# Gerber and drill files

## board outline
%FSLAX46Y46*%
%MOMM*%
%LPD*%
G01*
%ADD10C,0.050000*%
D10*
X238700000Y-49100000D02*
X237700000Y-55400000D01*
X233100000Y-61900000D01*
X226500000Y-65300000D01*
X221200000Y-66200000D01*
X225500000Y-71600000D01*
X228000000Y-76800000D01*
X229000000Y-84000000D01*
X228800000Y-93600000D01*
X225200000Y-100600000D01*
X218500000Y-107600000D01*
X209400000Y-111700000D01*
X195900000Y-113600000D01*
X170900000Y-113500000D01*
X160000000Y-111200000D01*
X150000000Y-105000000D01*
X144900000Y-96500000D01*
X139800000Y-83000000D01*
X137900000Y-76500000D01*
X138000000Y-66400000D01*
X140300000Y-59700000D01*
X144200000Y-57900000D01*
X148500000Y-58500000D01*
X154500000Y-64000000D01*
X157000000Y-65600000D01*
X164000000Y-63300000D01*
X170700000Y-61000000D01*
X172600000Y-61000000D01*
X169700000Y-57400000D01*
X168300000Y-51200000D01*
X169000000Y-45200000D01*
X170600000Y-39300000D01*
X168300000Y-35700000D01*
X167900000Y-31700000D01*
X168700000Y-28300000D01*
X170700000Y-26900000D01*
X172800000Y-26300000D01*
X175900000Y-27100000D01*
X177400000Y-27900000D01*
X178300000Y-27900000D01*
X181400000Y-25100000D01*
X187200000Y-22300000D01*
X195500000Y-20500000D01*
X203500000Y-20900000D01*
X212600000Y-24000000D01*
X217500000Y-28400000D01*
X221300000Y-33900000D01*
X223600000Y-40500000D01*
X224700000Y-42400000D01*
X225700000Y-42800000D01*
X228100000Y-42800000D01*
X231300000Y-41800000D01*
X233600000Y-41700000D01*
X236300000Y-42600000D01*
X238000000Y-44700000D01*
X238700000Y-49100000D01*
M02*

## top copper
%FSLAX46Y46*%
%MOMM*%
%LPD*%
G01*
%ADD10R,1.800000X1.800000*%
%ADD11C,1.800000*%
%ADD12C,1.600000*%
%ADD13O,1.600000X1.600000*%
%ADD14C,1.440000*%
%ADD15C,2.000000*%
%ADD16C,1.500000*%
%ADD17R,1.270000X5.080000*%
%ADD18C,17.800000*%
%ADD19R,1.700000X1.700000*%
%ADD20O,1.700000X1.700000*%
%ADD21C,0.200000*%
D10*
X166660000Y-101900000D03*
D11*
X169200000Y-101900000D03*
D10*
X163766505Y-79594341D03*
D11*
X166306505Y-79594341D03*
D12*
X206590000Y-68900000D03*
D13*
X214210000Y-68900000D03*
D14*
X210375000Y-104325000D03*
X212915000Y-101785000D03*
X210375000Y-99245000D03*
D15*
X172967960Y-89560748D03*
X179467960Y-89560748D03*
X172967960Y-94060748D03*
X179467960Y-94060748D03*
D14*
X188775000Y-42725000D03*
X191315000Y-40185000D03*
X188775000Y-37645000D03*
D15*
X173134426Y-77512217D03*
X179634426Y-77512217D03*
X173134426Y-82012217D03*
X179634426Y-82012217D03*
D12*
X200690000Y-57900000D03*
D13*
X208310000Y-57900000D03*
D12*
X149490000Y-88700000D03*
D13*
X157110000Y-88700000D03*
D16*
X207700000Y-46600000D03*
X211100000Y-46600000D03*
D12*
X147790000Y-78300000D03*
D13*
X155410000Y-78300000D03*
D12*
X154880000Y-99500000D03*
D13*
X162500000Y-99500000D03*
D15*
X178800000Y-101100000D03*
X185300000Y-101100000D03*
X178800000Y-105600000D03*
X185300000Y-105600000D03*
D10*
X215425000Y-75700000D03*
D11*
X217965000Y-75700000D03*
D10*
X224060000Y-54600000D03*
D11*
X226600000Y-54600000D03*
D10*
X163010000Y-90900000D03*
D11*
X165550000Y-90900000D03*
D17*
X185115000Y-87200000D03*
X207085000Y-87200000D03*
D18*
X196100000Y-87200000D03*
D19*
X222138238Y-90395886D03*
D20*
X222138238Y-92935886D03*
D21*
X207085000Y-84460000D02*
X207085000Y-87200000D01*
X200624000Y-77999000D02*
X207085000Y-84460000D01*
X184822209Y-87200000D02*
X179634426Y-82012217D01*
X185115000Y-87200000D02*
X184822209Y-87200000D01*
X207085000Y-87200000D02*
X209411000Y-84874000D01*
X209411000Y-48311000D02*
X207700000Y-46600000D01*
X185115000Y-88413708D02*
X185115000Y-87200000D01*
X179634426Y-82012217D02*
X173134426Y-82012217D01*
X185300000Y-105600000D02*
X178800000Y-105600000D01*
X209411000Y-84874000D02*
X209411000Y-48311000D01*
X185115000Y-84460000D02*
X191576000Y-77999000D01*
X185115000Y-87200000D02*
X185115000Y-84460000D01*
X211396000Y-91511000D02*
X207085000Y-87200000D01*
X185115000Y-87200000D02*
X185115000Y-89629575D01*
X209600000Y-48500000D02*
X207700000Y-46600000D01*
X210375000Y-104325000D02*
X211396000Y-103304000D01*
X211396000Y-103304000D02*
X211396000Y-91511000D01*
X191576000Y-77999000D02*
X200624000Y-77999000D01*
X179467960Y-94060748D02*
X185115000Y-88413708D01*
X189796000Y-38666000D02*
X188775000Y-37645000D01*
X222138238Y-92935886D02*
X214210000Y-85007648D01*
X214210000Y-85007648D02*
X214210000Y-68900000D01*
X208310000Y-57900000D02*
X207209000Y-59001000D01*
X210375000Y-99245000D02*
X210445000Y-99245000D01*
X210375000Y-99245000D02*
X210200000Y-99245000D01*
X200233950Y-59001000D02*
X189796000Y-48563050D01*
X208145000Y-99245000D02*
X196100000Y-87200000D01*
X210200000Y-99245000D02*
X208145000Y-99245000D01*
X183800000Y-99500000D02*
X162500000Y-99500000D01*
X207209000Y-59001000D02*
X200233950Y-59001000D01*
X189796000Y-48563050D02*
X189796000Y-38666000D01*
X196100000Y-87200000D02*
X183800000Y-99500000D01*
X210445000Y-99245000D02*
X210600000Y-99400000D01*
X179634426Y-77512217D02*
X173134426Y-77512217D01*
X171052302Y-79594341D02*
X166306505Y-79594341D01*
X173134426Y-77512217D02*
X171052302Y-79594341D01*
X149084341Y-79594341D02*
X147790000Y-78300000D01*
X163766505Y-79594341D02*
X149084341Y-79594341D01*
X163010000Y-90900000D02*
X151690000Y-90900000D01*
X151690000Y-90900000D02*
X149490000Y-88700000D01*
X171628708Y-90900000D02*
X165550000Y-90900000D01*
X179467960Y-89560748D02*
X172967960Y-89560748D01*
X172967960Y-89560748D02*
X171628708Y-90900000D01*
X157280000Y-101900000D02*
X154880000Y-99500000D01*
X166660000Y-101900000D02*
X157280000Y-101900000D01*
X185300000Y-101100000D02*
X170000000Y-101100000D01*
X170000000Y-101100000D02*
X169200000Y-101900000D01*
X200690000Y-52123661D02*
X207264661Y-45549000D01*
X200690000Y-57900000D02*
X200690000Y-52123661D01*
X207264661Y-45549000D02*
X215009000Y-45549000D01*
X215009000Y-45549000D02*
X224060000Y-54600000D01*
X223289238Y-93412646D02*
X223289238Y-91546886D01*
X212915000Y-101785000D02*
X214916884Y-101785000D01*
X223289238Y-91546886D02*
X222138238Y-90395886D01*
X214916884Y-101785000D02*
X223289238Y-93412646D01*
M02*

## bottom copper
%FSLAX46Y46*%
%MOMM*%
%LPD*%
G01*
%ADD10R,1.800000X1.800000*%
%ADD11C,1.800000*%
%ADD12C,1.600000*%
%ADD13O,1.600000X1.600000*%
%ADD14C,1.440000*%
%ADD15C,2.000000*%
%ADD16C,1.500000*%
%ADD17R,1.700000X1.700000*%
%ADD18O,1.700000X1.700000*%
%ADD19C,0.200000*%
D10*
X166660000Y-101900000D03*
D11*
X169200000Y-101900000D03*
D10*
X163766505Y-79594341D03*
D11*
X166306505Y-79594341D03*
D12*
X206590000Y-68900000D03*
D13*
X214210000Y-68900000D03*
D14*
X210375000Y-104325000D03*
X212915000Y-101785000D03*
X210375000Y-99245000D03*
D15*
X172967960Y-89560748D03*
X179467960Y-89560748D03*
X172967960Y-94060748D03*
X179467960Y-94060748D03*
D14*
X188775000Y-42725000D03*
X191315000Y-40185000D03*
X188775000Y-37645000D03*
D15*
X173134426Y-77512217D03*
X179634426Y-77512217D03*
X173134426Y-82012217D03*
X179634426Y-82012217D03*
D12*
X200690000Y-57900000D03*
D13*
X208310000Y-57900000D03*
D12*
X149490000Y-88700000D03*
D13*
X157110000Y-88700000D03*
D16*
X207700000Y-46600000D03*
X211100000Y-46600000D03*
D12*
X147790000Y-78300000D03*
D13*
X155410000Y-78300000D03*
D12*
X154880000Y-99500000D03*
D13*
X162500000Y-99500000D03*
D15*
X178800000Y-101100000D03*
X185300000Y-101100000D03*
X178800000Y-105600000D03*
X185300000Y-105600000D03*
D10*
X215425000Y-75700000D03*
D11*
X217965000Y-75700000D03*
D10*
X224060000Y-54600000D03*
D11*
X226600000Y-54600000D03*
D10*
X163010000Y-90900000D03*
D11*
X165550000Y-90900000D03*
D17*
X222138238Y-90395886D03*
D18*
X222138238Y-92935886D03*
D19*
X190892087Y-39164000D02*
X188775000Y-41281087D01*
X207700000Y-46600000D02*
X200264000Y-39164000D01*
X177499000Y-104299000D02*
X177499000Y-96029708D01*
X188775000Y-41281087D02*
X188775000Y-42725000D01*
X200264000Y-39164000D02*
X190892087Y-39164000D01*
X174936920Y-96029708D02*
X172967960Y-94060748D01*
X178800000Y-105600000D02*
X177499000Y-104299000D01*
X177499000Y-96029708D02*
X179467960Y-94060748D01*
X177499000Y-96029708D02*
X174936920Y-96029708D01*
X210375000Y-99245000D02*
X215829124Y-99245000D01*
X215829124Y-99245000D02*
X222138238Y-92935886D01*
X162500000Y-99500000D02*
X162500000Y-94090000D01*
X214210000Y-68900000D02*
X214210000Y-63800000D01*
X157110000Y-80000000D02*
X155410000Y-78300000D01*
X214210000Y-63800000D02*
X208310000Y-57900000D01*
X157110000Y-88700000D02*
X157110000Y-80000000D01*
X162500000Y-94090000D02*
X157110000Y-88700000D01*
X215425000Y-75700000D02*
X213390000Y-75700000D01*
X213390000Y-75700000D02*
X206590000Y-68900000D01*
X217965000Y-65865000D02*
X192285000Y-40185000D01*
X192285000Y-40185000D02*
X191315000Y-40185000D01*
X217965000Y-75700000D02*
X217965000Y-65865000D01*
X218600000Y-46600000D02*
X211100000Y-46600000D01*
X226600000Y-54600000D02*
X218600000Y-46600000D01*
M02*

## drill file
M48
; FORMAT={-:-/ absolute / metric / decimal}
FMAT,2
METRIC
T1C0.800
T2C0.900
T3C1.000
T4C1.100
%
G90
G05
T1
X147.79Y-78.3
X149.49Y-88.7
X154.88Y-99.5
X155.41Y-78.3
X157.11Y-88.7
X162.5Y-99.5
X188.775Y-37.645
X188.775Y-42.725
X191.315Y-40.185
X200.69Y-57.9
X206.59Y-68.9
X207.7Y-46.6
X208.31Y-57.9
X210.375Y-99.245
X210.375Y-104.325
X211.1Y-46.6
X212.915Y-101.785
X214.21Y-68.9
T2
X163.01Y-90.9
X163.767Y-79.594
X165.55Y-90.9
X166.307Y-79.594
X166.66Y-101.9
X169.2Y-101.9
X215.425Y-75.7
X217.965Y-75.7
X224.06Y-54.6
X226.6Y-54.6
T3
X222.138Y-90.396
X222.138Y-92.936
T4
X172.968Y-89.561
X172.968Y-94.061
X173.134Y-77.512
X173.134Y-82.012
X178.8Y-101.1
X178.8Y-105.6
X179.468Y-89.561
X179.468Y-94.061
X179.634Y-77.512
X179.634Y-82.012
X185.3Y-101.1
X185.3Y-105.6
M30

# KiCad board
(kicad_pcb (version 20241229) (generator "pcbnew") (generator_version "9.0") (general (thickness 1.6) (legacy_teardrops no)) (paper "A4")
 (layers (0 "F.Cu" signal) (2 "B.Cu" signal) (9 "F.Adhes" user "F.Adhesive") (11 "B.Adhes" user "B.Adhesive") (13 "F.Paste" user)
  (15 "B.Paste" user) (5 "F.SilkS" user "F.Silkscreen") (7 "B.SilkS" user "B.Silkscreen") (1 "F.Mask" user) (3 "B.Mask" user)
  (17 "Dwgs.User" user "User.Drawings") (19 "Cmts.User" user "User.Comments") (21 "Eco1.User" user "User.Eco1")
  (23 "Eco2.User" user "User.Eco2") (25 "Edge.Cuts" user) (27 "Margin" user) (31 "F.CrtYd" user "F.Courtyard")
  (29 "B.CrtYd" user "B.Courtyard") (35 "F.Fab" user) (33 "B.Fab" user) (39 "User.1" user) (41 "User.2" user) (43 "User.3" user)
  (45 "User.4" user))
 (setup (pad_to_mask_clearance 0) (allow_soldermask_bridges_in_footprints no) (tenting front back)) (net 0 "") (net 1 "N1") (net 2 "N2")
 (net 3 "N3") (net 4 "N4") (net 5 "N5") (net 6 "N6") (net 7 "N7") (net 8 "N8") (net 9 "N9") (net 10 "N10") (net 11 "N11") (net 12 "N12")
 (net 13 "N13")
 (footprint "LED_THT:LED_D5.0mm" (layer "F.Cu") (at 166.66 101.9)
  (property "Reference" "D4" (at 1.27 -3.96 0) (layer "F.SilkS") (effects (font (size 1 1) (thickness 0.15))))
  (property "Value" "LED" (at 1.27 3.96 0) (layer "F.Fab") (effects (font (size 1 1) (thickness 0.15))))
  (pad "1" thru_hole rect (at 0 0) (size 1.8 1.8) (drill 0.9) (layers "*.Cu" "*.Mask") (remove_unused_layers no) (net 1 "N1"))
  (pad "2" thru_hole circle (at 2.54 0) (size 1.8 1.8) (drill 0.9) (layers "*.Cu" "*.Mask") (remove_unused_layers no) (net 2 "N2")))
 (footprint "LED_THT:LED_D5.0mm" (layer "F.Cu") (at 163.766505 79.594341)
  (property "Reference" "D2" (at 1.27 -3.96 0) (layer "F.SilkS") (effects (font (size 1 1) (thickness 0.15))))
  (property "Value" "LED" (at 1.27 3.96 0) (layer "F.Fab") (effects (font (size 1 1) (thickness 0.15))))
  (pad "1" thru_hole rect (at 0 0) (size 1.8 1.8) (drill 0.9) (layers "*.Cu" "*.Mask") (remove_unused_layers no) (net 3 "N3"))
  (pad "2" thru_hole circle (at 2.54 0) (size 1.8 1.8) (drill 0.9) (layers "*.Cu" "*.Mask") (remove_unused_layers no) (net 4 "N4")))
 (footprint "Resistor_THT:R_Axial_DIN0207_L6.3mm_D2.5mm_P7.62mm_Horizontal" (layer "F.Cu") (at 206.59 68.9)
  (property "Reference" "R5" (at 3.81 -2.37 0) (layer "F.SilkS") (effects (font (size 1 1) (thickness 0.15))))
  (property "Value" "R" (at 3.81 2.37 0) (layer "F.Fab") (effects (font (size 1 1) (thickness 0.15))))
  (pad "1" thru_hole circle (at 0 0) (size 1.6 1.6) (drill 0.8) (layers "*.Cu" "*.Mask") (remove_unused_layers no) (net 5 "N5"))
  (pad "2" thru_hole oval (at 7.62 0) (size 1.6 1.6) (drill 0.8) (layers "*.Cu" "*.Mask") (remove_unused_layers no) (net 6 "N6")))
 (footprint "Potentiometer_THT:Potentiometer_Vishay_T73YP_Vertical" (layer "F.Cu") (at 210.375 104.325)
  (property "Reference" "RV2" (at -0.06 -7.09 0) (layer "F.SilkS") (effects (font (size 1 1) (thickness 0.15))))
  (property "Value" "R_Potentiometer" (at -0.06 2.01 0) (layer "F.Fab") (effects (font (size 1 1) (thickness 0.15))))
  (pad "1" thru_hole circle (at 0 0) (size 1.44 1.44) (drill 0.8) (layers "*.Cu" "*.Mask") (remove_unused_layers no) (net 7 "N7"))
  (pad "2" thru_hole circle (at 2.54 -2.54) (size 1.44 1.44) (drill 0.8) (layers "*.Cu" "*.Mask") (remove_unused_layers no) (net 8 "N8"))
  (pad "3" thru_hole circle (at 0 -5.08) (size 1.44 1.44) (drill 0.8) (layers "*.Cu" "*.Mask") (remove_unused_layers no) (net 6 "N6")))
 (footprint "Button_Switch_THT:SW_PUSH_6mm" (layer "F.Cu") (at 172.96796 89.560748)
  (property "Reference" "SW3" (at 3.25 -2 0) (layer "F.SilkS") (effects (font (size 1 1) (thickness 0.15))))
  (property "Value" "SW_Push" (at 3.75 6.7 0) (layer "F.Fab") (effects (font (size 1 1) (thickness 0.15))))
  (pad "1" thru_hole circle (at 0 0 90) (size 2 2) (drill 1.1) (layers "*.Cu" "*.Mask") (remove_unused_layers no) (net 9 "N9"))
  (pad "1" thru_hole circle (at 6.5 0 90) (size 2 2) (drill 1.1) (layers "*.Cu" "*.Mask") (remove_unused_layers no) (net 9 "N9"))
  (pad "2" thru_hole circle (at 0 4.5 90) (size 2 2) (drill 1.1) (layers "*.Cu" "*.Mask") (remove_unused_layers no) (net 7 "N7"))
  (pad "2" thru_hole circle (at 6.5 4.5 90) (size 2 2) (drill 1.1) (layers "*.Cu" "*.Mask") (remove_unused_layers no) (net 7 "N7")))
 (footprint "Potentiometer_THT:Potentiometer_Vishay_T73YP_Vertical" (layer "F.Cu") (at 188.775 42.725)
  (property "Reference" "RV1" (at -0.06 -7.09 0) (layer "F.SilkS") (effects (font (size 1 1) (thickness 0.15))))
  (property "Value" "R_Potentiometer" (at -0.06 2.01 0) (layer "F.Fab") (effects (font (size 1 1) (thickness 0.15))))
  (pad "1" thru_hole circle (at 0 0) (size 1.44 1.44) (drill 0.8) (layers "*.Cu" "*.Mask") (remove_unused_layers no) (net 7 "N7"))
  (pad "2" thru_hole circle (at 2.54 -2.54) (size 1.44 1.44) (drill 0.8) (layers "*.Cu" "*.Mask") (remove_unused_layers no) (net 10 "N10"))
  (pad "3" thru_hole circle (at 0 -5.08) (size 1.44 1.44) (drill 0.8) (layers "*.Cu" "*.Mask") (remove_unused_layers no) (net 6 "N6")))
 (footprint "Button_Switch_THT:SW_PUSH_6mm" (layer "F.Cu") (at 173.134426 77.512217)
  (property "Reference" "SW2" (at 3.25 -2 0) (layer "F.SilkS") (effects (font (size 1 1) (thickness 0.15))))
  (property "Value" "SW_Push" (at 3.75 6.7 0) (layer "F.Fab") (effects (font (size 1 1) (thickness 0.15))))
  (pad "1" thru_hole circle (at 0 0 90) (size 2 2) (drill 1.1) (layers "*.Cu" "*.Mask") (remove_unused_layers no) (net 4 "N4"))
  (pad "1" thru_hole circle (at 6.5 0 90) (size 2 2) (drill 1.1) (layers "*.Cu" "*.Mask") (remove_unused_layers no) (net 4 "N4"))
  (pad "2" thru_hole circle (at 0 4.5 90) (size 2 2) (drill 1.1) (layers "*.Cu" "*.Mask") (remove_unused_layers no) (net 7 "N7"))
  (pad "2" thru_hole circle (at 6.5 4.5 90) (size 2 2) (drill 1.1) (layers "*.Cu" "*.Mask") (remove_unused_layers no) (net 7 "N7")))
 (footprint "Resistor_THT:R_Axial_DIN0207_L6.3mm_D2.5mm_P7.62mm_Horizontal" (layer "F.Cu") (at 200.69 57.9)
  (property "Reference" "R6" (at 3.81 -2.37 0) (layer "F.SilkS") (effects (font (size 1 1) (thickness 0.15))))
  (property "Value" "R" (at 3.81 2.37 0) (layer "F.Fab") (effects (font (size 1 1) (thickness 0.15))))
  (pad "1" thru_hole circle (at 0 0) (size 1.6 1.6) (drill 0.8) (layers "*.Cu" "*.Mask") (remove_unused_layers no) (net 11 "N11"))
  (pad "2" thru_hole oval (at 7.62 0) (size 1.6 1.6) (drill 0.8) (layers "*.Cu" "*.Mask") (remove_unused_layers no) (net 6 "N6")))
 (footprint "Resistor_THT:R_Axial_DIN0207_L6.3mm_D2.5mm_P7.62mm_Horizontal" (layer "F.Cu") (at 149.49 88.7)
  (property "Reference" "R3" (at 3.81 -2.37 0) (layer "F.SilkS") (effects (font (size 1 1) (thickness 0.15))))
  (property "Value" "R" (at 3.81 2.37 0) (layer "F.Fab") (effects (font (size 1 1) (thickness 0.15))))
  (pad "1" thru_hole circle (at 0 0) (size 1.6 1.6) (drill 0.8) (layers "*.Cu" "*.Mask") (remove_unused_layers no) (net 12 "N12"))
  (pad "2" thru_hole oval (at 7.62 0) (size 1.6 1.6) (drill 0.8) (layers "*.Cu" "*.Mask") (remove_unused_layers no) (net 6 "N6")))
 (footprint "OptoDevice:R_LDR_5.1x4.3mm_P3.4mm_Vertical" (layer "F.Cu") (at 207.7 46.6)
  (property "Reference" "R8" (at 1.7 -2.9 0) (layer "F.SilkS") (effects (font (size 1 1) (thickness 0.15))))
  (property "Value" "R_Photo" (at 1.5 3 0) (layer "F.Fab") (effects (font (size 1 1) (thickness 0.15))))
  (pad "1" thru_hole circle (at 0 0) (size 1.5 1.5) (drill 0.8) (layers "*.Cu" "*.Mask") (remove_unused_layers no) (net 7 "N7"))
  (pad "2" thru_hole circle (at 3.4 0) (size 1.5 1.5) (drill 0.8) (layers "*.Cu" "*.Mask") (remove_unused_layers no) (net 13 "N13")))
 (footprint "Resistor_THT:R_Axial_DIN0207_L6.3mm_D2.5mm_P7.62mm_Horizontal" (layer "F.Cu") (at 147.79 78.3)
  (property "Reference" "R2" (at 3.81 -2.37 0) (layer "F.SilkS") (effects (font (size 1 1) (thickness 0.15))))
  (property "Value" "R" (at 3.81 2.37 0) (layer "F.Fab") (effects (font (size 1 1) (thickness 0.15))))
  (pad "1" thru_hole circle (at 0 0) (size 1.6 1.6) (drill 0.8) (layers "*.Cu" "*.Mask") (remove_unused_layers no) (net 3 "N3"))
  (pad "2" thru_hole oval (at 7.62 0) (size 1.6 1.6) (drill 0.8) (layers "*.Cu" "*.Mask") (remove_unused_layers no) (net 6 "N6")))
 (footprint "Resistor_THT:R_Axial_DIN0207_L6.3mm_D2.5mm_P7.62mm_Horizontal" (layer "F.Cu") (at 154.88 99.5)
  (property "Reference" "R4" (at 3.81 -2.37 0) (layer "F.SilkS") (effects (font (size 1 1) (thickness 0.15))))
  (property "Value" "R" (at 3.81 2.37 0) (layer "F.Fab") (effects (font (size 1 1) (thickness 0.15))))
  (pad "1" thru_hole circle (at 0 0) (size 1.6 1.6) (drill 0.8) (layers "*.Cu" "*.Mask") (remove_unused_layers no) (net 1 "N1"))
  (pad "2" thru_hole oval (at 7.62 0) (size 1.6 1.6) (drill 0.8) (layers "*.Cu" "*.Mask") (remove_unused_layers no) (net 6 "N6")))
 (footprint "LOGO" (layer "F.Cu") (at 189.1 67.6)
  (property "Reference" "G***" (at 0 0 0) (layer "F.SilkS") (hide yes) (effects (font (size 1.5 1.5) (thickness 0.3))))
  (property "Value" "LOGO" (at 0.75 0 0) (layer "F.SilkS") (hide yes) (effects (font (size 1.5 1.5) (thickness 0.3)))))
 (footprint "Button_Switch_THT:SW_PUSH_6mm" (layer "F.Cu") (at 178.8 101.1)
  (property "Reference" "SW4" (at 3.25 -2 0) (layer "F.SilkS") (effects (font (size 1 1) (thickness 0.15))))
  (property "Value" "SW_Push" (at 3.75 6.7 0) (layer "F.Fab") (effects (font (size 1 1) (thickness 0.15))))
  (pad "1" thru_hole circle (at 0 0 90) (size 2 2) (drill 1.1) (layers "*.Cu" "*.Mask") (remove_unused_layers no) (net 2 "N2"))
  (pad "1" thru_hole circle (at 6.5 0 90) (size 2 2) (drill 1.1) (layers "*.Cu" "*.Mask") (remove_unused_layers no) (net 2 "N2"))
  (pad "2" thru_hole circle (at 0 4.5 90) (size 2 2) (drill 1.1) (layers "*.Cu" "*.Mask") (remove_unused_layers no) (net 7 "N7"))
  (pad "2" thru_hole circle (at 6.5 4.5 90) (size 2 2) (drill 1.1) (layers "*.Cu" "*.Mask") (remove_unused_layers no) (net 7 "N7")))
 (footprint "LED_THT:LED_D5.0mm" (layer "F.Cu") (at 215.425 75.7)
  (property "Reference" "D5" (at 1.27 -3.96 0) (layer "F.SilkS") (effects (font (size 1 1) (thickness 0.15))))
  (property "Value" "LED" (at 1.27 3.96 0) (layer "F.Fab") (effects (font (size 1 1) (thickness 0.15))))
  (pad "1" thru_hole rect (at 0 0) (size 1.8 1.8) (drill 0.9) (layers "*.Cu" "*.Mask") (remove_unused_layers no) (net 5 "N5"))
  (pad "2" thru_hole circle (at 2.54 0) (size 1.8 1.8) (drill 0.9) (layers "*.Cu" "*.Mask") (remove_unused_layers no) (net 10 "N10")))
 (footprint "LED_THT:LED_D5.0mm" (layer "F.Cu") (at 224.06 54.6)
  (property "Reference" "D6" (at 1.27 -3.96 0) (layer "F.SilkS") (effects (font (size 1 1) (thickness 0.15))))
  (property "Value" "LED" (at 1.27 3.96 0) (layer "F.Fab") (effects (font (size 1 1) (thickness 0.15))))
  (pad "1" thru_hole rect (at 0 0) (size 1.8 1.8) (drill 0.9) (layers "*.Cu" "*.Mask") (remove_unused_layers no) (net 11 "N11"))
  (pad "2" thru_hole circle (at 2.54 0) (size 1.8 1.8) (drill 0.9) (layers "*.Cu" "*.Mask") (remove_unused_layers no) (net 13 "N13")))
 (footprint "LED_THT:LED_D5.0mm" (layer "F.Cu") (at 163.01 90.9)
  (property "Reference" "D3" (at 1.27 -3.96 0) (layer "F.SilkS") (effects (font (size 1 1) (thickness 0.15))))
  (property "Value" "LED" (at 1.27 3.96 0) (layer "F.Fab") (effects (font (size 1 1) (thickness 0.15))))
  (pad "1" thru_hole rect (at 0 0) (size 1.8 1.8) (drill 0.9) (layers "*.Cu" "*.Mask") (remove_unused_layers no) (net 12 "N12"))
  (pad "2" thru_hole circle (at 2.54 0) (size 1.8 1.8) (drill 0.9) (layers "*.Cu" "*.Mask") (remove_unused_layers no) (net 9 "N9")))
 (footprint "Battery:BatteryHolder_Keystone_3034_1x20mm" (layer "F.Cu") (at 196.1 87.2)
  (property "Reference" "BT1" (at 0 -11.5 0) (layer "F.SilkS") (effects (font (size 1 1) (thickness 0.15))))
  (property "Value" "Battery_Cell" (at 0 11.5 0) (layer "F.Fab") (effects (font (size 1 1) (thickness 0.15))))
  (pad "1" smd rect (at -10.985 0) (size 1.27 5.08) (layers "F.Cu" "F.Mask" "F.Paste") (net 7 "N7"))
  (pad "1" smd rect (at 10.985 0) (size 1.27 5.08) (layers "F.Cu" "F.Mask" "F.Paste") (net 7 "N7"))
  (pad "2" smd circle (at 0 0) (size 17.8 17.8) (layers "F.Cu" "F.Mask") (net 6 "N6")))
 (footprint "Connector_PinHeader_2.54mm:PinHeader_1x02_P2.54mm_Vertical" (layer "F.Cu") (at 222.138238 90.395886)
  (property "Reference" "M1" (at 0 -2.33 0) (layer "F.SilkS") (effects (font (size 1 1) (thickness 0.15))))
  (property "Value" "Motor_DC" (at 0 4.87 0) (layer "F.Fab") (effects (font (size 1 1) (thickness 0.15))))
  (pad "1" thru_hole rect (at 0 0) (size 1.7 1.7) (drill 1) (layers "*.Cu" "*.Mask") (remove_unused_layers no) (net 8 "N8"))
  (pad "2" thru_hole oval (at 0 2.54) (size 1.7 1.7) (drill 1) (layers "*.Cu" "*.Mask") (remove_unused_layers no) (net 6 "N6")))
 (gr_poly
  (pts (xy 238.7 49.1) (xy 237.7 55.4) (xy 233.1 61.9) (xy 226.5 65.3) (xy 221.2 66.2) (xy 225.5 71.6) (xy 228 76.8) (xy 229 84)
   (xy 228.8 93.6) (xy 225.2 100.6) (xy 218.5 107.6) (xy 209.4 111.7) (xy 195.9 113.6) (xy 170.9 113.5) (xy 160 111.2) (xy 150 105)
   (xy 144.9 96.5) (xy 139.8 83) (xy 137.9 76.5) (xy 138 66.4) (xy 140.3 59.7) (xy 144.2 57.9) (xy 148.5 58.5) (xy 154.5 64) (xy 157 65.6)
   (xy 164 63.3) (xy 170.7 61) (xy 172.6 61) (xy 169.7 57.4) (xy 168.3 51.2) (xy 169 45.2) (xy 170.6 39.3) (xy 168.3 35.7) (xy 167.9 31.7)
   (xy 168.7 28.3) (xy 170.7 26.9) (xy 172.8 26.3) (xy 175.9 27.1) (xy 177.4 27.9) (xy 178.3 27.9) (xy 181.4 25.1) (xy 187.2 22.3)
   (xy 195.5 20.5) (xy 203.5 20.9) (xy 212.6 24) (xy 217.5 28.4) (xy 221.3 33.9) (xy 223.6 40.5) (xy 224.7 42.4) (xy 225.7 42.8)
   (xy 228.1 42.8) (xy 231.3 41.8) (xy 233.6 41.7) (xy 236.3 42.6) (xy 238 44.7))
  (stroke (width 0.05) (type solid)) (fill no) (layer "Edge.Cuts"))
 (segment (start 207.085 84.46) (end 207.085 87.2) (width 0.2) (layer "F.Cu") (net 7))
 (segment (start 200.624 77.999) (end 207.085 84.46) (width 0.2) (layer "F.Cu") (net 7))
 (segment (start 184.822209 87.2) (end 179.634426 82.012217) (width 0.2) (layer "F.Cu") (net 7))
 (segment (start 185.115 87.2) (end 184.822209 87.2) (width 0.2) (layer "F.Cu") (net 7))
 (segment (start 207.085 87.2) (end 209.411 84.874) (width 0.2) (layer "F.Cu") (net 7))
 (segment (start 209.411 48.311) (end 207.7 46.6) (width 0.2) (layer "F.Cu") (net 7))
 (segment (start 185.115 88.413708) (end 185.115 87.2) (width 0.2) (layer "F.Cu") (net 7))
 (segment (start 179.634426 82.012217) (end 173.134426 82.012217) (width 0.2) (layer "F.Cu") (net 7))
 (segment (start 185.3 105.6) (end 178.8 105.6) (width 0.2) (layer "F.Cu") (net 7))
 (segment (start 209.411 84.874) (end 209.411 48.311) (width 0.2) (layer "F.Cu") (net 7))
 (segment (start 185.115 84.46) (end 191.576 77.999) (width 0.2) (layer "F.Cu") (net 7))
 (segment (start 185.115 87.2) (end 185.115 84.46) (width 0.2) (layer "F.Cu") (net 7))
 (segment (start 211.396 91.511) (end 207.085 87.2) (width 0.2) (layer "F.Cu") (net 7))
 (segment (start 185.115 87.2) (end 185.115 89.629575) (width 0.2) (layer "F.Cu") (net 7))
 (segment (start 209.6 48.5) (end 207.7 46.6) (width 0.2) (layer "F.Cu") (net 7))
 (segment (start 210.375 104.325) (end 211.396 103.304) (width 0.2) (layer "F.Cu") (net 7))
 (segment (start 211.396 103.304) (end 211.396 91.511) (width 0.2) (layer "F.Cu") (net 7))
 (segment (start 191.576 77.999) (end 200.624 77.999) (width 0.2) (layer "F.Cu") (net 7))
 (segment (start 179.46796 94.060748) (end 185.115 88.413708) (width 0.2) (layer "F.Cu") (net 7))
 (segment (start 190.892087 39.164) (end 188.775 41.281087) (width 0.2) (layer "B.Cu") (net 7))
 (segment (start 207.7 46.6) (end 200.264 39.164) (width 0.2) (layer "B.Cu") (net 7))
 (segment (start 177.499 104.299) (end 177.499 96.029708) (width 0.2) (layer "B.Cu") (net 7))
 (segment (start 188.775 41.281087) (end 188.775 42.725) (width 0.2) (layer "B.Cu") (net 7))
 (segment (start 200.264 39.164) (end 190.892087 39.164) (width 0.2) (layer "B.Cu") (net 7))
 (segment (start 174.93692 96.029708) (end 172.96796 94.060748) (width 0.2) (layer "B.Cu") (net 7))
 (segment (start 178.8 105.6) (end 177.499 104.299) (width 0.2) (layer "B.Cu") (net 7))
 (segment (start 177.499 96.029708) (end 179.46796 94.060748) (width 0.2) (layer "B.Cu") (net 7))
 (segment (start 177.499 96.029708) (end 174.93692 96.029708) (width 0.2) (layer "B.Cu") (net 7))
 (segment (start 189.796 38.666) (end 188.775 37.645) (width 0.2) (layer "F.Cu") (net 6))
 (segment (start 222.138238 92.935886) (end 214.21 85.007648) (width 0.2) (layer "F.Cu") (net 6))
 (segment (start 214.21 85.007648) (end 214.21 68.9) (width 0.2) (layer "F.Cu") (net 6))
 (segment (start 208.31 57.9) (end 207.209 59.001) (width 0.2) (layer "F.Cu") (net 6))
 (segment (start 210.375 99.245) (end 210.445 99.245) (width 0.2) (layer "F.Cu") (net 6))
 (segment (start 210.375 99.245) (end 210.2 99.245) (width 0.2) (layer "F.Cu") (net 6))
 (segment (start 200.23395 59.001) (end 189.796 48.56305) (width 0.2) (layer "F.Cu") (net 6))
 (segment (start 208.145 99.245) (end 196.1 87.2) (width 0.2) (layer "F.Cu") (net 6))
 (segment (start 210.2 99.245) (end 208.145 99.245) (width 0.2) (layer "F.Cu") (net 6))
 (segment (start 183.8 99.5) (end 162.5 99.5) (width 0.2) (layer "F.Cu") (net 6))
 (segment (start 207.209 59.001) (end 200.23395 59.001) (width 0.2) (layer "F.Cu") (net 6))
 (segment (start 189.796 48.56305) (end 189.796 38.666) (width 0.2) (layer "F.Cu") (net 6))
 (segment (start 196.1 87.2) (end 183.8 99.5) (width 0.2) (layer "F.Cu") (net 6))
 (segment (start 210.445 99.245) (end 210.6 99.4) (width 0.2) (layer "F.Cu") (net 6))
 (segment (start 210.375 99.245) (end 215.829124 99.245) (width 0.2) (layer "B.Cu") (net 6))
 (segment (start 215.829124 99.245) (end 222.138238 92.935886) (width 0.2) (layer "B.Cu") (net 6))
 (segment (start 162.5 99.5) (end 162.5 94.09) (width 0.2) (layer "B.Cu") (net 6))
 (segment (start 214.21 68.9) (end 214.21 63.8) (width 0.2) (layer "B.Cu") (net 6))
 (segment (start 157.11 80) (end 155.41 78.3) (width 0.2) (layer "B.Cu") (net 6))
 (segment (start 214.21 63.8) (end 208.31 57.9) (width 0.2) (layer "B.Cu") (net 6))
 (segment (start 157.11 88.7) (end 157.11 80) (width 0.2) (layer "B.Cu") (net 6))
 (segment (start 162.5 94.09) (end 157.11 88.7) (width 0.2) (layer "B.Cu") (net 6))
 (segment (start 179.634426 77.512217) (end 173.134426 77.512217) (width 0.2) (layer "F.Cu") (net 4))
 (segment (start 171.052302 79.594341) (end 166.306505 79.594341) (width 0.2) (layer "F.Cu") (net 4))
 (segment (start 173.134426 77.512217) (end 171.052302 79.594341) (width 0.2) (layer "F.Cu") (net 4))
 (segment (start 149.084341 79.594341) (end 147.79 78.3) (width 0.2) (layer "F.Cu") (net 3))
 (segment (start 163.766505 79.594341) (end 149.084341 79.594341) (width 0.2) (layer "F.Cu") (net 3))
 (segment (start 163.01 90.9) (end 151.69 90.9) (width 0.2) (layer "F.Cu") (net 12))
 (segment (start 151.69 90.9) (end 149.49 88.7) (width 0.2) (layer "F.Cu") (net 12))
 (segment (start 171.628708 90.9) (end 165.55 90.9) (width 0.2) (layer "F.Cu") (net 9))
 (segment (start 179.46796 89.560748) (end 172.96796 89.560748) (width 0.2) (layer "F.Cu") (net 9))
 (segment (start 172.96796 89.560748) (end 171.628708 90.9) (width 0.2) (layer "F.Cu") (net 9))
 (segment (start 157.28 101.9) (end 154.88 99.5) (width 0.2) (layer "F.Cu") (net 1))
 (segment (start 166.66 101.9) (end 157.28 101.9) (width 0.2) (layer "F.Cu") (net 1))
 (segment (start 185.3 101.1) (end 170 101.1) (width 0.2) (layer "F.Cu") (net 2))
 (segment (start 170 101.1) (end 169.2 101.9) (width 0.2) (layer "F.Cu") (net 2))
 (segment (start 215.425 75.7) (end 213.39 75.7) (width 0.2) (layer "B.Cu") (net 5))
 (segment (start 213.39 75.7) (end 206.59 68.9) (width 0.2) (layer "B.Cu") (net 5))
 (segment (start 217.965 65.865) (end 192.285 40.185) (width 0.2) (layer "B.Cu") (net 10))
 (segment (start 192.285 40.185) (end 191.315 40.185) (width 0.2) (layer "B.Cu") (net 10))
 (segment (start 217.965 75.7) (end 217.965 65.865) (width 0.2) (layer "B.Cu") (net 10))
 (segment (start 218.6 46.6) (end 211.1 46.6) (width 0.2) (layer "B.Cu") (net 13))
 (segment (start 226.6 54.6) (end 218.6 46.6) (width 0.2) (layer "B.Cu") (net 13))
 (segment (start 200.69 52.123661) (end 207.264661 45.549) (width 0.2) (layer "F.Cu") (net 11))
 (segment (start 200.69 57.9) (end 200.69 52.123661) (width 0.2) (layer "F.Cu") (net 11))
 (segment (start 207.264661 45.549) (end 215.009 45.549) (width 0.2) (layer "F.Cu") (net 11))
 (segment (start 215.009 45.549) (end 224.06 54.6) (width 0.2) (layer "F.Cu") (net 11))
 (segment (start 223.289238 93.412646) (end 223.289238 91.546886) (width 0.2) (layer "F.Cu") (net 8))
 (segment (start 212.915 101.785) (end 214.916884 101.785) (width 0.2) (layer "F.Cu") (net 8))
 (segment (start 223.289238 91.546886) (end 222.138238 90.395886) (width 0.2) (layer "F.Cu") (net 8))
 (segment (start 214.916884 101.785) (end 223.289238 93.412646) (width 0.2) (layer "F.Cu") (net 8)))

